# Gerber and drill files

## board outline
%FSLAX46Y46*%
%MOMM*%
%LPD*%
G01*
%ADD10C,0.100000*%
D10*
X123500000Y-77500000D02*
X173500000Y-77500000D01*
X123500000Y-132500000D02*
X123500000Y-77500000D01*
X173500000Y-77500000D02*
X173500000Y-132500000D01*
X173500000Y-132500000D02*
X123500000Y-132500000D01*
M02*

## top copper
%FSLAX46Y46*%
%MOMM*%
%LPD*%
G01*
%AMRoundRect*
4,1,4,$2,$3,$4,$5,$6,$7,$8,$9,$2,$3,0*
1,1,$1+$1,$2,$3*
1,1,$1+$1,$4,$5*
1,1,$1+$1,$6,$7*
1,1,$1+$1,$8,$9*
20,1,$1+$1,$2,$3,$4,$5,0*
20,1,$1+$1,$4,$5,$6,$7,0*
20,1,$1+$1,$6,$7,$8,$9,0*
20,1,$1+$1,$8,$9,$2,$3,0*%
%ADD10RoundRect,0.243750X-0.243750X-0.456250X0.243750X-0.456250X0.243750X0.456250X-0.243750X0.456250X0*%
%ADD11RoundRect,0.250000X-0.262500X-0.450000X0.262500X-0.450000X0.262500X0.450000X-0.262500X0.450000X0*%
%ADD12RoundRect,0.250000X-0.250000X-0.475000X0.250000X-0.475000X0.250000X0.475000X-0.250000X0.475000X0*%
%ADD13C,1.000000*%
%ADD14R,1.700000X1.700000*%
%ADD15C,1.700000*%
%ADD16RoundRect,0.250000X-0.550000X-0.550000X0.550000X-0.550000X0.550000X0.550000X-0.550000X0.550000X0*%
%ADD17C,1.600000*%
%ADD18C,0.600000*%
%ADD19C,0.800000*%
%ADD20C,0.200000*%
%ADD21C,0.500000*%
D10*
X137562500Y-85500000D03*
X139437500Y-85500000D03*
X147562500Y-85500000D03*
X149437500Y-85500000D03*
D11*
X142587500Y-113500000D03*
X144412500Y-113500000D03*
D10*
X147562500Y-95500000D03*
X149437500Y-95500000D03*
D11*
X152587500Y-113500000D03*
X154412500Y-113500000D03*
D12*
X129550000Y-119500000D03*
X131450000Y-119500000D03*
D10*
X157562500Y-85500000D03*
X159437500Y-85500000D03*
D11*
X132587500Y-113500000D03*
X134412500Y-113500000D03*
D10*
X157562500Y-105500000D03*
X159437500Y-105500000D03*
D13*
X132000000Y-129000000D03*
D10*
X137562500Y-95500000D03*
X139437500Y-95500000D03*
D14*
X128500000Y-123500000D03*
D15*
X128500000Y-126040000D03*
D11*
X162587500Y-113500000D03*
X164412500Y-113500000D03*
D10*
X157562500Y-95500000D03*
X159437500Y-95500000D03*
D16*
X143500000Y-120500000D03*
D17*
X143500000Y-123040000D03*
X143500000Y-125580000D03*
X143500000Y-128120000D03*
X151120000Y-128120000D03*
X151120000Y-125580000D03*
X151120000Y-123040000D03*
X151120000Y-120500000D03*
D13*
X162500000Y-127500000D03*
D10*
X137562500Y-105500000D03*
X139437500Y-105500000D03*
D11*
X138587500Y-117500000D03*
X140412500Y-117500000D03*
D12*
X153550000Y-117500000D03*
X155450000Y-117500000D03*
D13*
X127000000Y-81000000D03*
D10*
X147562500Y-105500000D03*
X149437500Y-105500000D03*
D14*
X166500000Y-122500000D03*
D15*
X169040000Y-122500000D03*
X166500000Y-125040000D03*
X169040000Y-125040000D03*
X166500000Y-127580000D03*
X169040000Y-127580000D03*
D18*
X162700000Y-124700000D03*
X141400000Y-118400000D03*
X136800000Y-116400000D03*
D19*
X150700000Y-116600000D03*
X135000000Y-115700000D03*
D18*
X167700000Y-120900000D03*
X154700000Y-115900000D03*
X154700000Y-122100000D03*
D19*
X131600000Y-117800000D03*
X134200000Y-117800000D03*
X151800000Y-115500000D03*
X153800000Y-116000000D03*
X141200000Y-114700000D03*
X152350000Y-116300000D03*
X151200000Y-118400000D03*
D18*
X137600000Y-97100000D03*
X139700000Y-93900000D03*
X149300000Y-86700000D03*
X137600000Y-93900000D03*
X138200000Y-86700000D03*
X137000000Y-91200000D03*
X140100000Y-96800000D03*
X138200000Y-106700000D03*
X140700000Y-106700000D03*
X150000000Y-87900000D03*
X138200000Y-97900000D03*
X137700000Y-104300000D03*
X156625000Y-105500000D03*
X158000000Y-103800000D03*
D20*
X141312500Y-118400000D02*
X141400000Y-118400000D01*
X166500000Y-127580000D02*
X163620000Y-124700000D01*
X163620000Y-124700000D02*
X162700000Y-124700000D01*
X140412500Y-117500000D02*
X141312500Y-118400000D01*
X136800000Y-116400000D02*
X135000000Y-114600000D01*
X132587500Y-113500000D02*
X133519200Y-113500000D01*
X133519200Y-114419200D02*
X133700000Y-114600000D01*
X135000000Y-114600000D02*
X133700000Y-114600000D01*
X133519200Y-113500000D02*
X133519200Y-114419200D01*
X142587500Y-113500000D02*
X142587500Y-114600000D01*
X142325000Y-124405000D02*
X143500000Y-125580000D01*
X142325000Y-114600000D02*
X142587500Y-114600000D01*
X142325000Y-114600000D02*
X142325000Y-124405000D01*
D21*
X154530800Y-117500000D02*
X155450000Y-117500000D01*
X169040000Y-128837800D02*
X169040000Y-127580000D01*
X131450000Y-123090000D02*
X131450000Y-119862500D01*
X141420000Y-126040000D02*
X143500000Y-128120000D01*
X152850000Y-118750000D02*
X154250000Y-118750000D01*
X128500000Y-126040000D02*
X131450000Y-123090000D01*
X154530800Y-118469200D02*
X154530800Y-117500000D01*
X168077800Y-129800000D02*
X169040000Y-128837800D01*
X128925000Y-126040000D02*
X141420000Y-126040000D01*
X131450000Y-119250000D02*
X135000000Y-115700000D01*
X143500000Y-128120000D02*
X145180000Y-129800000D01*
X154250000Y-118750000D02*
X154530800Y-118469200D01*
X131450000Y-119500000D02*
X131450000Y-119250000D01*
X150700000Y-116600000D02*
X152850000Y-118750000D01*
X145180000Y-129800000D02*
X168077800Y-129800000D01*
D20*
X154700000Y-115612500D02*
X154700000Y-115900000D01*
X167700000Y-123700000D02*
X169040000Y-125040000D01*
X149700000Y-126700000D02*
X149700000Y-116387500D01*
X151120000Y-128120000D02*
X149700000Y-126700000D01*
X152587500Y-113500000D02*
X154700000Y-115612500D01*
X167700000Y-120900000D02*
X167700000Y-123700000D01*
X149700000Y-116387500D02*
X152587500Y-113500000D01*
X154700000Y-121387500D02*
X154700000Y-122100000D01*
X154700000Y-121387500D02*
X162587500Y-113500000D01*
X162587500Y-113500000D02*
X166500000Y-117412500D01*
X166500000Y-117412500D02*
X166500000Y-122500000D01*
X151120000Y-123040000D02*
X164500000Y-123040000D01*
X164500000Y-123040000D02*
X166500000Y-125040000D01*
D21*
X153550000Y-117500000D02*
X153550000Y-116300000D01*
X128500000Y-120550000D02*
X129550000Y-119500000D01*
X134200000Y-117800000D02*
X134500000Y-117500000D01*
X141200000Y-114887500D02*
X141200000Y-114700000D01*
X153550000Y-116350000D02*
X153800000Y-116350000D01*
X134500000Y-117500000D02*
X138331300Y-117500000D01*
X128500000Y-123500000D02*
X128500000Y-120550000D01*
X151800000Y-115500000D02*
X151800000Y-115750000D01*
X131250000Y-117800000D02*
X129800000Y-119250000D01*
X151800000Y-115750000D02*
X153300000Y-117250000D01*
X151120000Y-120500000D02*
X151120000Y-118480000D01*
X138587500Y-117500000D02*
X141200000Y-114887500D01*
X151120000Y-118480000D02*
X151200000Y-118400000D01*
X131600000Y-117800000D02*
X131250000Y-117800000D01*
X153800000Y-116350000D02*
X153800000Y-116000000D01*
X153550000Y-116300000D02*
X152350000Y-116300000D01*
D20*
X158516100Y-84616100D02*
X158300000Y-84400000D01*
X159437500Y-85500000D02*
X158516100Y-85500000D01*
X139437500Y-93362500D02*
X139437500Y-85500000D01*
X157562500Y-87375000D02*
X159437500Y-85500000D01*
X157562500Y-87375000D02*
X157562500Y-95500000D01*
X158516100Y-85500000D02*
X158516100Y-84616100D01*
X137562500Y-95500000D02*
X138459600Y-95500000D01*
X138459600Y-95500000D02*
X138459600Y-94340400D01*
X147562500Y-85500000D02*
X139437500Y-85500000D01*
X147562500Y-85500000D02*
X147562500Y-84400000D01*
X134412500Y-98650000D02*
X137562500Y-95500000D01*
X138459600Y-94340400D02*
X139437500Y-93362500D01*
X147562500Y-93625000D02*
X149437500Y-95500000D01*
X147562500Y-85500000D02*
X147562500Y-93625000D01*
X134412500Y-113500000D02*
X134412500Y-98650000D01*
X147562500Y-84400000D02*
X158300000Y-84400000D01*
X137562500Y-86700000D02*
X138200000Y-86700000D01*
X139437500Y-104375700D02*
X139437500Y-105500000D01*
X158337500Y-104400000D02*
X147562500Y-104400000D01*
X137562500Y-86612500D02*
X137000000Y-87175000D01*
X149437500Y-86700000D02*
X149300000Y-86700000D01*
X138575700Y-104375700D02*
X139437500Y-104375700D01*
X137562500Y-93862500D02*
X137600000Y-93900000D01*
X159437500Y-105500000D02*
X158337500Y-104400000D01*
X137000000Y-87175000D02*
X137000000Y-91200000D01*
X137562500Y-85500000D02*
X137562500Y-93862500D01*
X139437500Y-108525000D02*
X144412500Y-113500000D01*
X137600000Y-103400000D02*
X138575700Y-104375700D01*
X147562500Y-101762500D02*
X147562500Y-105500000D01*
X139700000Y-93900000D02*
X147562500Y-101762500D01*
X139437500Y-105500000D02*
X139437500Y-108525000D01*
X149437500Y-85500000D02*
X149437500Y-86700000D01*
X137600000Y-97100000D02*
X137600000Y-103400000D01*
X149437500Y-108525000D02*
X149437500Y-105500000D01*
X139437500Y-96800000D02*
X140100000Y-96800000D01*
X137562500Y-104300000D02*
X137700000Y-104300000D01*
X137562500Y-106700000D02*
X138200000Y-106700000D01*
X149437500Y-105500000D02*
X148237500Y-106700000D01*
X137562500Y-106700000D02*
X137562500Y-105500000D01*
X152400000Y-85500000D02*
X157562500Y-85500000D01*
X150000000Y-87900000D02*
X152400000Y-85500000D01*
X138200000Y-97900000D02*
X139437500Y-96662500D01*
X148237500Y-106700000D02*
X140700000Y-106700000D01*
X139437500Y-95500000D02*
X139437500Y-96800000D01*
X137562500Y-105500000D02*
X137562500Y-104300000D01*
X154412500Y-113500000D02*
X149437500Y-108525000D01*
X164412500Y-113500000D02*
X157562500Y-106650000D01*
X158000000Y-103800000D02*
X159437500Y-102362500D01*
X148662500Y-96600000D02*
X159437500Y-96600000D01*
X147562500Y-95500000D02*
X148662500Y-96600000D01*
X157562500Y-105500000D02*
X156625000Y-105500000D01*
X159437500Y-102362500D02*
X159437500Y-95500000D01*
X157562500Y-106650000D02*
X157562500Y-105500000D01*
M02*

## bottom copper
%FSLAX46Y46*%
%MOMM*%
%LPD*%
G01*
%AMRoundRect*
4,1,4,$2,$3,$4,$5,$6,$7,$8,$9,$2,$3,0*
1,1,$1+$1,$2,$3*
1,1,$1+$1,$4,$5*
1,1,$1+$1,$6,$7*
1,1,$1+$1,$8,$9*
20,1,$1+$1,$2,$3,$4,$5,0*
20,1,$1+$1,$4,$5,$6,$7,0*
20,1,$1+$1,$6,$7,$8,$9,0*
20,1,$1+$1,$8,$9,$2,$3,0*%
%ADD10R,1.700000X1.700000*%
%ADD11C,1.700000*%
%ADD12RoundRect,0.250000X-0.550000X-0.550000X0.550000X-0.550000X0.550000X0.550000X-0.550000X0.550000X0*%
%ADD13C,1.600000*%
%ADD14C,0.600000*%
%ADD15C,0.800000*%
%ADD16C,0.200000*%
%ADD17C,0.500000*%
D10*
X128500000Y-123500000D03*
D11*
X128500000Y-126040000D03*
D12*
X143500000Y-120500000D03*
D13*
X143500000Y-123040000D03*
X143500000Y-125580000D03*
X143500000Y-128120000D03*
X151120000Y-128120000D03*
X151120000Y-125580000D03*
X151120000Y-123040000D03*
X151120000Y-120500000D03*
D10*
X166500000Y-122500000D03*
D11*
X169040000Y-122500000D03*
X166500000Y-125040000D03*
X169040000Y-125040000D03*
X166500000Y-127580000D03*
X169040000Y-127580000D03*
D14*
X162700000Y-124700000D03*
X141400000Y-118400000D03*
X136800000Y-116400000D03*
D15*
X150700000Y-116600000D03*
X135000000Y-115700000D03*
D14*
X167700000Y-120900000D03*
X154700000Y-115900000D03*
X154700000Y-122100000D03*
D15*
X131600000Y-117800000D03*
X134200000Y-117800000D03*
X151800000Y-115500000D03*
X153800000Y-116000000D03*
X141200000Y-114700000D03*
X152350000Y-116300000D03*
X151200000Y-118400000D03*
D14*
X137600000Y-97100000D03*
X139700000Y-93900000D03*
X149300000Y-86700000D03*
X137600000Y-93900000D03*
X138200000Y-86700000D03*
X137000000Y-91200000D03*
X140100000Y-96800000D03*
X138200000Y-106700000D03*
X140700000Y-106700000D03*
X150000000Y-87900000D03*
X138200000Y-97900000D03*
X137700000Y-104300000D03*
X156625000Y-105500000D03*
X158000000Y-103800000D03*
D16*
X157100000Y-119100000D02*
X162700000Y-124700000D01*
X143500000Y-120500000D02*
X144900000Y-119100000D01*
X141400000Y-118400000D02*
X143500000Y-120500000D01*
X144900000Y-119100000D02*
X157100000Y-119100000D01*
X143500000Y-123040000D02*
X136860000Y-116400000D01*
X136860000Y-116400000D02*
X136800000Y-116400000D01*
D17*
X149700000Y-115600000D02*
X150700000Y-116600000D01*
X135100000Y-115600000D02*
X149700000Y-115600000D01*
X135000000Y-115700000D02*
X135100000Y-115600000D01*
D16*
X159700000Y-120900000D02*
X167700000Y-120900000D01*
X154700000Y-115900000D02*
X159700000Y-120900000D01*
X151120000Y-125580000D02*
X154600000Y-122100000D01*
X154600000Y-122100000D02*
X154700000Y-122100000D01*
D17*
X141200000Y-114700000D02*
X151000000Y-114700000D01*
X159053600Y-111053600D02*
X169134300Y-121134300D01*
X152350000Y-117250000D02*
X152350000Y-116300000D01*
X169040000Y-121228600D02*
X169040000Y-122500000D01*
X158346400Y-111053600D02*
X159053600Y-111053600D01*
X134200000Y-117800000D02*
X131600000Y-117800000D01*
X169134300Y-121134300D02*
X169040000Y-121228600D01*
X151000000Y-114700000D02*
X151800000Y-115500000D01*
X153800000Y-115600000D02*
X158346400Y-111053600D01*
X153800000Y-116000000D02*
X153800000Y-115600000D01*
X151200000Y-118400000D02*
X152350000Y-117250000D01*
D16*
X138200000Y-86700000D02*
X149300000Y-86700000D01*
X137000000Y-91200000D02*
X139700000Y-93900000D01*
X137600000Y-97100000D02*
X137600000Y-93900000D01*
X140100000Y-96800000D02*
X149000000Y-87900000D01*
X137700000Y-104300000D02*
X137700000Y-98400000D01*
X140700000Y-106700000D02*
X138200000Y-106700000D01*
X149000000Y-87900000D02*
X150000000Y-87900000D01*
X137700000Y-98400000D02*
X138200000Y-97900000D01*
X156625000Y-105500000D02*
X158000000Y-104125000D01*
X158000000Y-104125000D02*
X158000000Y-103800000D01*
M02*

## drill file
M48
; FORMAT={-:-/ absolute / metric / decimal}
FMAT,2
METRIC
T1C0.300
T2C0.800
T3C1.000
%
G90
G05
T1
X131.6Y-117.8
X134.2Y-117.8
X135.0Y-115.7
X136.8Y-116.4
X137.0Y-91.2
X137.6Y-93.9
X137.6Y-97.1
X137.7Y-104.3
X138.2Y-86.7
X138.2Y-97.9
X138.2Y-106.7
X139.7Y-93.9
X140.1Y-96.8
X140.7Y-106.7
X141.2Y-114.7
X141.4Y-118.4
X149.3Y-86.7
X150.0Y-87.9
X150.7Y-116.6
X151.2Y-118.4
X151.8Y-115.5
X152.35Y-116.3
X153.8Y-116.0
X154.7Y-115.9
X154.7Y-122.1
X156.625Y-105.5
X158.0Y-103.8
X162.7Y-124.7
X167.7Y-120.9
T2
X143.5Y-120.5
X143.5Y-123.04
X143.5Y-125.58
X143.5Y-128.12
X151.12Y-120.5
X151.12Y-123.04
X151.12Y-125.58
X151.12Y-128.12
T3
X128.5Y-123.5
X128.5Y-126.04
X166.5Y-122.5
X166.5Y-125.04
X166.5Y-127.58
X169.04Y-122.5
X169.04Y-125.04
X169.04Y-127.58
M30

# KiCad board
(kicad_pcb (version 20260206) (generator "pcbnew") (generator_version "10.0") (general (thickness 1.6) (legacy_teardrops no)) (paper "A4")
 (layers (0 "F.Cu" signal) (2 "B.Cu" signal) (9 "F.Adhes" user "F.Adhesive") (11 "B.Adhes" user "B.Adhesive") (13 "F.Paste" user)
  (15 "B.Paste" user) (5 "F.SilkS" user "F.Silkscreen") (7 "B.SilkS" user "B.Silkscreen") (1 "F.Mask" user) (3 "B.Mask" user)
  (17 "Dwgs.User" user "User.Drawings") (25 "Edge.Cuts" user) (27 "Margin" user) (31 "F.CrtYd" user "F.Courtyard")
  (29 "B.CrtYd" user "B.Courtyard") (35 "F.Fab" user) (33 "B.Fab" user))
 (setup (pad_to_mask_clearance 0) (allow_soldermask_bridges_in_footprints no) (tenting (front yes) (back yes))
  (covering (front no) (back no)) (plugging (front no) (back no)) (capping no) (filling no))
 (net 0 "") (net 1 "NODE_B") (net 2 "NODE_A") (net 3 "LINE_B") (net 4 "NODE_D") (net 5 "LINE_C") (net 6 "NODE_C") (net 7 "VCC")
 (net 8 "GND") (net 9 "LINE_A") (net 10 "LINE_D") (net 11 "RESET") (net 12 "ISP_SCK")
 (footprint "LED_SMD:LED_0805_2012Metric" (layer "F.Cu") (at 138.5 85.5)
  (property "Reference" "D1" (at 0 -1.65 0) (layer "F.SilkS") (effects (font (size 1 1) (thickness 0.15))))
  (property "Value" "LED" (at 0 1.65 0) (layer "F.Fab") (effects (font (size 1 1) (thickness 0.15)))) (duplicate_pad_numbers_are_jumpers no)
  (pad "1" smd roundrect (at -0.9375 0) (size 0.975 1.4) (layers "F.Cu" "F.Mask" "F.Paste") (roundrect_rratio 0.25) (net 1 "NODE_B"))
  (pad "2" smd roundrect (at 0.9375 0) (size 0.975 1.4) (layers "F.Cu" "F.Mask" "F.Paste") (roundrect_rratio 0.25) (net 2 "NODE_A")))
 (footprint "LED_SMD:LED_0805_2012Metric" (layer "F.Cu") (at 148.5 85.5)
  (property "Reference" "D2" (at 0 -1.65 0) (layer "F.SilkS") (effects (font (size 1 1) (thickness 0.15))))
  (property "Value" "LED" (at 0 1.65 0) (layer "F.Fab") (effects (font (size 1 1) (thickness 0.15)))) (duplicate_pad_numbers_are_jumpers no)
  (pad "1" smd roundrect (at -0.9375 0) (size 0.975 1.4) (layers "F.Cu" "F.Mask" "F.Paste") (roundrect_rratio 0.25) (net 2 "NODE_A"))
  (pad "2" smd roundrect (at 0.9375 0) (size 0.975 1.4) (layers "F.Cu" "F.Mask" "F.Paste") (roundrect_rratio 0.25) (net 1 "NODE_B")))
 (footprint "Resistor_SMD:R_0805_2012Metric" (layer "F.Cu") (at 143.5 113.5)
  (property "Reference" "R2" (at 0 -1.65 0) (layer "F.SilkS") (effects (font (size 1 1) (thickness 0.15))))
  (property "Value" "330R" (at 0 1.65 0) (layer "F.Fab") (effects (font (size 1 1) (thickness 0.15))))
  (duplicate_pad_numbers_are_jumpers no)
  (pad "1" smd roundrect (at -0.9125 0) (size 1.025 1.4) (layers "F.Cu" "F.Mask" "F.Paste") (roundrect_rratio 0.243902) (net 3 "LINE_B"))
  (pad "2" smd roundrect (at 0.9125 0) (size 1.025 1.4) (layers "F.Cu" "F.Mask" "F.Paste") (roundrect_rratio 0.243902) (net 1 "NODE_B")))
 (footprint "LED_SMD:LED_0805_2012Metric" (layer "F.Cu") (at 148.5 95.5)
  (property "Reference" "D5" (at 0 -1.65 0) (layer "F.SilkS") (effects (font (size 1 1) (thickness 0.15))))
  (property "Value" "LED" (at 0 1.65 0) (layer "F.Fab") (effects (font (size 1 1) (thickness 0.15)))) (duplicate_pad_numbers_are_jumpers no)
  (pad "1" smd roundrect (at -0.9375 0) (size 0.975 1.4) (layers "F.Cu" "F.Mask" "F.Paste") (roundrect_rratio 0.25) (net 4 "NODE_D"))
  (pad "2" smd roundrect (at 0.9375 0) (size 0.975 1.4) (layers "F.Cu" "F.Mask" "F.Paste") (roundrect_rratio 0.25) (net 2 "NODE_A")))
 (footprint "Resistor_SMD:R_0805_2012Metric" (layer "F.Cu") (at 153.5 113.5)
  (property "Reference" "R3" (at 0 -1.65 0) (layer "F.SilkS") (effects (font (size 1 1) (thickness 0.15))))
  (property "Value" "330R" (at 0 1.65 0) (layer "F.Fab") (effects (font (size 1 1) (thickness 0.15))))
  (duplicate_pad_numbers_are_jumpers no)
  (pad "1" smd roundrect (at -0.9125 0) (size 1.025 1.4) (layers "F.Cu" "F.Mask" "F.Paste") (roundrect_rratio 0.243902) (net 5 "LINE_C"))
  (pad "2" smd roundrect (at 0.9125 0) (size 1.025 1.4) (layers "F.Cu" "F.Mask" "F.Paste") (roundrect_rratio 0.243902) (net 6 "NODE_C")))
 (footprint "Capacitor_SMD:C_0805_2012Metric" (layer "F.Cu") (at 130.5 119.5)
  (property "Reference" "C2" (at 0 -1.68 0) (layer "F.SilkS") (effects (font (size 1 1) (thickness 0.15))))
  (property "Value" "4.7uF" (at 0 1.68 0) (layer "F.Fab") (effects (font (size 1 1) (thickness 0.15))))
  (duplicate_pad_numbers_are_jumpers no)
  (pad "1" smd roundrect (at -0.95 0) (size 1 1.45) (layers "F.Cu" "F.Mask" "F.Paste") (roundrect_rratio 0.25) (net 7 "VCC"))
  (pad "2" smd roundrect (at 0.95 0) (size 1 1.45) (layers "F.Cu" "F.Mask" "F.Paste") (roundrect_rratio 0.25) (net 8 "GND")))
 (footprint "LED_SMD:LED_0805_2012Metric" (layer "F.Cu") (at 158.5 85.5)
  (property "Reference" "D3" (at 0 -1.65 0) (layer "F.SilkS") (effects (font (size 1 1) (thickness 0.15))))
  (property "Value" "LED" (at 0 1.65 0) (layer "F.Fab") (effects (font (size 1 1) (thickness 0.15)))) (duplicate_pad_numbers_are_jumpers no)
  (pad "1" smd roundrect (at -0.9375 0) (size 0.975 1.4) (layers "F.Cu" "F.Mask" "F.Paste") (roundrect_rratio 0.25) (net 6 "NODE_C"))
  (pad "2" smd roundrect (at 0.9375 0) (size 0.975 1.4) (layers "F.Cu" "F.Mask" "F.Paste") (roundrect_rratio 0.25) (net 2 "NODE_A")))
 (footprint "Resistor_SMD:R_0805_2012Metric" (layer "F.Cu") (at 133.5 113.5)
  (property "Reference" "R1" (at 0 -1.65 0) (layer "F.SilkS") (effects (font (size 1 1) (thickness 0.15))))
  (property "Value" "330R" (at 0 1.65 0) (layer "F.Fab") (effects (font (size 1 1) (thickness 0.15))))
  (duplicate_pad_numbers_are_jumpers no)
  (pad "1" smd roundrect (at -0.9125 0) (size 1.025 1.4) (layers "F.Cu" "F.Mask" "F.Paste") (roundrect_rratio 0.243902) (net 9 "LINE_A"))
  (pad "2" smd roundrect (at 0.9125 0) (size 1.025 1.4) (layers "F.Cu" "F.Mask" "F.Paste") (roundrect_rratio 0.243902) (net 2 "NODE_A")))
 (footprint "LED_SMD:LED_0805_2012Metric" (layer "F.Cu") (at 158.5 105.5)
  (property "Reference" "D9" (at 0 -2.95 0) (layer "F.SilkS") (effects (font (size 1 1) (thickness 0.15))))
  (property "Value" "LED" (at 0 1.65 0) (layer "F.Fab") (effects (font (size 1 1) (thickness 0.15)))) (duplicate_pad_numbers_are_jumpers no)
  (pad "1" smd roundrect (at -0.9375 0) (size 0.975 1.4) (layers "F.Cu" "F.Mask" "F.Paste") (roundrect_rratio 0.25) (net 4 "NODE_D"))
  (pad "2" smd roundrect (at 0.9375 0) (size 0.975 1.4) (layers "F.Cu" "F.Mask" "F.Paste") (roundrect_rratio 0.25) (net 1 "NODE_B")))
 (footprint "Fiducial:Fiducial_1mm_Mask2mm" (layer "F.Cu") (at 132 129)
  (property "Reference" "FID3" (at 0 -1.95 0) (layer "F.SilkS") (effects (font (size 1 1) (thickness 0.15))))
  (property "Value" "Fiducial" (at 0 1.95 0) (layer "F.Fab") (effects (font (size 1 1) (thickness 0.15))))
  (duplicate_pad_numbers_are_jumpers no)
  (pad "" smd circle (at 0 0) (size 1 1) (layers "F.Cu" "F.Mask") (solder_mask_margin 0.5) (clearance 0.6)))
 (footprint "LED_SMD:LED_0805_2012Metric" (layer "F.Cu") (at 138.5 95.5)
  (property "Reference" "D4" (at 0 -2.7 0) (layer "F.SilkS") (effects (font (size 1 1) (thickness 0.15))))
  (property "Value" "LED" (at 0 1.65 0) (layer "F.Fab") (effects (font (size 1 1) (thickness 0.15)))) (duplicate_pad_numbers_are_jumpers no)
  (pad "1" smd roundrect (at -0.9375 0) (size 0.975 1.4) (layers "F.Cu" "F.Mask" "F.Paste") (roundrect_rratio 0.25) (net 2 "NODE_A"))
  (pad "2" smd roundrect (at 0.9375 0) (size 0.975 1.4) (layers "F.Cu" "F.Mask" "F.Paste") (roundrect_rratio 0.25) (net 6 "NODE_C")))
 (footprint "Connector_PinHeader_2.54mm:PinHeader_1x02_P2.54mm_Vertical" (layer "F.Cu") (at 128.5 123.5)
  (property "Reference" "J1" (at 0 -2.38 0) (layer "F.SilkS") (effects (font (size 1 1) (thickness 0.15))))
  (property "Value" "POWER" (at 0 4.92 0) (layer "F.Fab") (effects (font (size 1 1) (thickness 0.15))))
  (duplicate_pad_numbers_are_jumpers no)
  (pad "1" thru_hole rect (at 0 0) (size 1.7 1.7) (drill 1) (layers "*.Cu" "*.Mask") (remove_unused_layers no) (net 7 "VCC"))
  (pad "2" thru_hole circle (at 0 2.54) (size 1.7 1.7) (drill 1) (layers "*.Cu" "*.Mask") (remove_unused_layers no) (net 8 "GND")))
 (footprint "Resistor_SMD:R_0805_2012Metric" (layer "F.Cu") (at 163.5 113.5)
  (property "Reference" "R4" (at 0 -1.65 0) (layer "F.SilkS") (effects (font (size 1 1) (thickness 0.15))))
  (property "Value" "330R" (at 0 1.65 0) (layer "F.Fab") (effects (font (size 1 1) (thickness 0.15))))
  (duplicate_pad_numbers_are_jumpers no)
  (pad "1" smd roundrect (at -0.9125 0) (size 1.025 1.4) (layers "F.Cu" "F.Mask" "F.Paste") (roundrect_rratio 0.243902) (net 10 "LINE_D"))
  (pad "2" smd roundrect (at 0.9125 0) (size 1.025 1.4) (layers "F.Cu" "F.Mask" "F.Paste") (roundrect_rratio 0.243902) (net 4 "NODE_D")))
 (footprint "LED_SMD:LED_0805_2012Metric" (layer "F.Cu") (at 158.5 95.5)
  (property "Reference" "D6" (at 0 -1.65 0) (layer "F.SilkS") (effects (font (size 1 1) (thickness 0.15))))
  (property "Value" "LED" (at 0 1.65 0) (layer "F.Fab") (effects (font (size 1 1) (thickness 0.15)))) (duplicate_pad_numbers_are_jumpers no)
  (pad "1" smd roundrect (at -0.9375 0) (size 0.975 1.4) (layers "F.Cu" "F.Mask" "F.Paste") (roundrect_rratio 0.25) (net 2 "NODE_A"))
  (pad "2" smd roundrect (at 0.9375 0) (size 0.975 1.4) (layers "F.Cu" "F.Mask" "F.Paste") (roundrect_rratio 0.25) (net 4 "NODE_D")))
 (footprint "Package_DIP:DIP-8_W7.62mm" (layer "F.Cu") (at 143.5 120.5)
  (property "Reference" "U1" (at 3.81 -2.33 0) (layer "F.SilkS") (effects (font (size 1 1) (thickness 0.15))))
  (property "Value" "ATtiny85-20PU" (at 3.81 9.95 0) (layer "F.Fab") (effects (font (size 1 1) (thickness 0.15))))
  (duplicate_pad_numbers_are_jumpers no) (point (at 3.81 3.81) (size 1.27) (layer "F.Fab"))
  (pad "1" thru_hole roundrect (at 0 0) (size 1.6 1.6) (drill 0.8) (layers "*.Cu" "*.Mask") (remove_unused_layers no)
   (roundrect_rratio 0.15625) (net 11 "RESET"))
  (pad "2" thru_hole circle (at 0 2.54) (size 1.6 1.6) (drill 0.8) (layers "*.Cu" "*.Mask") (remove_unused_layers no) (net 9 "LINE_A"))
  (pad "3" thru_hole circle (at 0 5.08) (size 1.6 1.6) (drill 0.8) (layers "*.Cu" "*.Mask") (remove_unused_layers no) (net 3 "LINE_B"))
  (pad "4" thru_hole circle (at 0 7.62) (size 1.6 1.6) (drill 0.8) (layers "*.Cu" "*.Mask") (remove_unused_layers no) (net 8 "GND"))
  (pad "5" thru_hole circle (at 7.62 7.62) (size 1.6 1.6) (drill 0.8) (layers "*.Cu" "*.Mask") (remove_unused_layers no) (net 5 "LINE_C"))
  (pad "6" thru_hole circle (at 7.62 5.08) (size 1.6 1.6) (drill 0.8) (layers "*.Cu" "*.Mask") (remove_unused_layers no) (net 10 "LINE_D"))
  (pad "7" thru_hole circle (at 7.62 2.54) (size 1.6 1.6) (drill 0.8) (layers "*.Cu" "*.Mask") (remove_unused_layers no) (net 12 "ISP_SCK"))
  (pad "8" thru_hole circle (at 7.62 0) (size 1.6 1.6) (drill 0.8) (layers "*.Cu" "*.Mask") (remove_unused_layers no) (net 7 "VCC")))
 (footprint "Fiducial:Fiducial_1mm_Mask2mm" (layer "F.Cu") (at 162.5 127.5)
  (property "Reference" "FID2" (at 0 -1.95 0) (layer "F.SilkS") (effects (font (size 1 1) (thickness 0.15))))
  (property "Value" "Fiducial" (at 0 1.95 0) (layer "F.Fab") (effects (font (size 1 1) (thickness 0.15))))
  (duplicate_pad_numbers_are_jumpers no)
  (pad "" smd circle (at 0 0) (size 1 1) (layers "F.Cu" "F.Mask") (solder_mask_margin 0.5) (clearance 0.6)))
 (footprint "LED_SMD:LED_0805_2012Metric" (layer "F.Cu") (at 138.5 105.5)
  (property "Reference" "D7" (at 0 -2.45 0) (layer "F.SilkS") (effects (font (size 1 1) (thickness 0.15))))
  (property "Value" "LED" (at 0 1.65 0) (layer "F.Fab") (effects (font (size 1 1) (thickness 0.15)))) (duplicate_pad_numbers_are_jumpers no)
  (pad "1" smd roundrect (at -0.9375 0) (size 0.975 1.4) (layers "F.Cu" "F.Mask" "F.Paste") (roundrect_rratio 0.25) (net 6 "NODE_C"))
  (pad "2" smd roundrect (at 0.9375 0) (size 0.975 1.4) (layers "F.Cu" "F.Mask" "F.Paste") (roundrect_rratio 0.25) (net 1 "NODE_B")))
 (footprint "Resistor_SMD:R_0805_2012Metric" (layer "F.Cu") (at 139.5 117.5)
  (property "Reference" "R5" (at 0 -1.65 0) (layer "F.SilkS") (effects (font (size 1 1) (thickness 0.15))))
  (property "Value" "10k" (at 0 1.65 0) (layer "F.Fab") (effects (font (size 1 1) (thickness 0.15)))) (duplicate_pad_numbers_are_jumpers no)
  (pad "1" smd roundrect (at -0.9125 0) (size 1.025 1.4) (layers "F.Cu" "F.Mask" "F.Paste") (roundrect_rratio 0.243902) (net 7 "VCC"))
  (pad "2" smd roundrect (at 0.9125 0) (size 1.025 1.4) (layers "F.Cu" "F.Mask" "F.Paste") (roundrect_rratio 0.243902) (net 11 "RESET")))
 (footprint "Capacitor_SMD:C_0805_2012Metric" (layer "F.Cu") (at 154.5 117.5)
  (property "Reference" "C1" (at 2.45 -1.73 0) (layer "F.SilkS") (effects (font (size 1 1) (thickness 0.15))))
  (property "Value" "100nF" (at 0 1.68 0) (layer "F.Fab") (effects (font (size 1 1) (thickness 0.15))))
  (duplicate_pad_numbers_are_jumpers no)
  (pad "1" smd roundrect (at -0.95 0) (size 1 1.45) (layers "F.Cu" "F.Mask" "F.Paste") (roundrect_rratio 0.25) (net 7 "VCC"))
  (pad "2" smd roundrect (at 0.95 0) (size 1 1.45) (layers "F.Cu" "F.Mask" "F.Paste") (roundrect_rratio 0.25) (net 8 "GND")))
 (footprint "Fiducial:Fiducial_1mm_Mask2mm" (layer "F.Cu") (at 127 81)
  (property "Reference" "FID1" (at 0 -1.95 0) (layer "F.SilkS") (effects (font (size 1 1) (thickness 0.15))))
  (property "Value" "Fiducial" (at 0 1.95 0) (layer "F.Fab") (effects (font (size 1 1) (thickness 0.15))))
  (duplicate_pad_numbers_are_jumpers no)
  (pad "" smd circle (at 0 0) (size 1 1) (layers "F.Cu" "F.Mask") (solder_mask_margin 0.5) (clearance 0.6)))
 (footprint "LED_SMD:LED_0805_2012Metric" (layer "F.Cu") (at 148.5 105.5)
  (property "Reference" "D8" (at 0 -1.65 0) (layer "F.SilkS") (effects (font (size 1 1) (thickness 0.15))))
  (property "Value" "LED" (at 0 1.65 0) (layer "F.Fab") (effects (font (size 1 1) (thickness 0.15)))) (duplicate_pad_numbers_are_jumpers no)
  (pad "1" smd roundrect (at -0.9375 0) (size 0.975 1.4) (layers "F.Cu" "F.Mask" "F.Paste") (roundrect_rratio 0.25) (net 1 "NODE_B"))
  (pad "2" smd roundrect (at 0.9375 0) (size 0.975 1.4) (layers "F.Cu" "F.Mask" "F.Paste") (roundrect_rratio 0.25) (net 6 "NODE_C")))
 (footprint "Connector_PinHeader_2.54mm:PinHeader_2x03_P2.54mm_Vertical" (layer "F.Cu") (at 166.5 122.5)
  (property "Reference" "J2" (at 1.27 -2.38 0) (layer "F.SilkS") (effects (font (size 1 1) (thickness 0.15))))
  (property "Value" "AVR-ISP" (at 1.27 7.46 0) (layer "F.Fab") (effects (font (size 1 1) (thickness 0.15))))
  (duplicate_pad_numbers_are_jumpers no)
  (pad "1" thru_hole rect (at 0 0) (size 1.7 1.7) (drill 1) (layers "*.Cu" "*.Mask") (remove_unused_layers no) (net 10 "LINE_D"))
  (pad "2" thru_hole circle (at 2.54 0) (size 1.7 1.7) (drill 1) (layers "*.Cu" "*.Mask") (remove_unused_layers no) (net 7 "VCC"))
  (pad "3" thru_hole circle (at 0 2.54) (size 1.7 1.7) (drill 1) (layers "*.Cu" "*.Mask") (remove_unused_layers no) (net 12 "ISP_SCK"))
  (pad "4" thru_hole circle (at 2.54 2.54) (size 1.7 1.7) (drill 1) (layers "*.Cu" "*.Mask") (remove_unused_layers no) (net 5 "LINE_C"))
  (pad "5" thru_hole circle (at 0 5.08) (size 1.7 1.7) (drill 1) (layers "*.Cu" "*.Mask") (remove_unused_layers no) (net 11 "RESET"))
  (pad "6" thru_hole circle (at 2.54 5.08) (size 1.7 1.7) (drill 1) (layers "*.Cu" "*.Mask") (remove_unused_layers no) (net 8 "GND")))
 (gr_line (start 123.5 77.5) (end 173.5 77.5) (stroke (width 0.1) (type default)) (layer "Edge.Cuts"))
 (gr_line (start 123.5 132.5) (end 123.5 77.5) (stroke (width 0.1) (type default)) (layer "Edge.Cuts"))
 (gr_line (start 173.5 77.5) (end 173.5 132.5) (stroke (width 0.1) (type default)) (layer "Edge.Cuts"))
 (gr_line (start 173.5 132.5) (end 123.5 132.5) (stroke (width 0.1) (type default)) (layer "Edge.Cuts"))
 (segment (start 141.3125 118.4) (end 141.4 118.4) (width 0.2) (layer "F.Cu") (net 11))
 (segment (start 166.5 127.58) (end 163.62 124.7) (width 0.2) (layer "F.Cu") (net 11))
 (segment (start 163.62 124.7) (end 162.7 124.7) (width 0.2) (layer "F.Cu") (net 11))
 (segment (start 140.4125 117.5) (end 141.3125 118.4) (width 0.2) (layer "F.Cu") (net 11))
 (via (at 162.7 124.7) (size 0.6) (drill 0.3) (layers "F.Cu" "B.Cu") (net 11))
 (via (at 141.4 118.4) (size 0.6) (drill 0.3) (layers "F.Cu" "B.Cu") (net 11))
 (segment (start 157.1 119.1) (end 162.7 124.7) (width 0.2) (layer "B.Cu") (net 11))
 (segment (start 143.5 120.5) (end 144.9 119.1) (width 0.2) (layer "B.Cu") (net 11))
 (segment (start 141.4 118.4) (end 143.5 120.5) (width 0.2) (layer "B.Cu") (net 11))
 (segment (start 144.9 119.1) (end 157.1 119.1) (width 0.2) (layer "B.Cu") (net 11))
 (segment (start 136.8 116.4) (end 135 114.6) (width 0.2) (layer "F.Cu") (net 9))
 (segment (start 132.5875 113.5) (end 133.5192 113.5) (width 0.2) (layer "F.Cu") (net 9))
 (segment (start 133.5192 114.4192) (end 133.7 114.6) (width 0.2) (layer "F.Cu") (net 9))
 (segment (start 135 114.6) (end 133.7 114.6) (width 0.2) (layer "F.Cu") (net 9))
 (segment (start 133.5192 113.5) (end 133.5192 114.4192) (width 0.2) (layer "F.Cu") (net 9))
 (via (at 136.8 116.4) (size 0.6) (drill 0.3) (layers "F.Cu" "B.Cu") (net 9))
 (segment (start 143.5 123.04) (end 136.86 116.4) (width 0.2) (layer "B.Cu") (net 9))
 (segment (start 136.86 116.4) (end 136.8 116.4) (width 0.2) (layer "B.Cu") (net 9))
 (segment (start 142.5875 113.5) (end 142.5875 114.6) (width 0.2) (layer "F.Cu") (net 3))
 (segment (start 142.325 124.405) (end 143.5 125.58) (width 0.2) (layer "F.Cu") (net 3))
 (segment (start 142.325 114.6) (end 142.5875 114.6) (width 0.2) (layer "F.Cu") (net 3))
 (segment (start 142.325 114.6) (end 142.325 124.405) (width 0.2) (layer "F.Cu") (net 3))
 (segment (start 154.5308 117.5) (end 155.45 117.5) (width 0.5) (layer "F.Cu") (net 8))
 (segment (start 169.04 128.8378) (end 169.04 127.58) (width 0.5) (layer "F.Cu") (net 8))
 (segment (start 131.45 123.09) (end 131.45 119.8625) (width 0.5) (layer "F.Cu") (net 8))
 (segment (start 141.42 126.04) (end 143.5 128.12) (width 0.5) (layer "F.Cu") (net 8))
 (segment (start 152.85 118.75) (end 154.25 118.75) (width 0.5) (layer "F.Cu") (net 8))
 (segment (start 128.5 126.04) (end 131.45 123.09) (width 0.5) (layer "F.Cu") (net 8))
 (segment (start 154.5308 118.4692) (end 154.5308 117.5) (width 0.5) (layer "F.Cu") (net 8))
 (segment (start 168.0778 129.8) (end 169.04 128.8378) (width 0.5) (layer "F.Cu") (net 8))
 (segment (start 128.925 126.04) (end 141.42 126.04) (width 0.5) (layer "F.Cu") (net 8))
 (segment (start 131.45 119.25) (end 135 115.7) (width 0.5) (layer "F.Cu") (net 8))
 (segment (start 143.5 128.12) (end 145.18 129.8) (width 0.5) (layer "F.Cu") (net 8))
 (segment (start 154.25 118.75) (end 154.5308 118.4692) (width 0.5) (layer "F.Cu") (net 8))
 (segment (start 131.45 119.5) (end 131.45 119.25) (width 0.5) (layer "F.Cu") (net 8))
 (segment (start 150.7 116.6) (end 152.85 118.75) (width 0.5) (layer "F.Cu") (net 8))
 (segment (start 145.18 129.8) (end 168.0778 129.8) (width 0.5) (layer "F.Cu") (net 8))
 (via (at 150.7 116.6) (size 0.8) (drill 0.3) (layers "F.Cu" "B.Cu") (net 8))
 (via (at 135 115.7) (size 0.8) (drill 0.3) (layers "F.Cu" "B.Cu") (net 8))
 (segment (start 149.7 115.6) (end 150.7 116.6) (width 0.5) (layer "B.Cu") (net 8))
 (segment (start 135.1 115.6) (end 149.7 115.6) (width 0.5) (layer "B.Cu") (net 8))
 (segment (start 135 115.7) (end 135.1 115.6) (width 0.5) (layer "B.Cu") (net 8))
 (segment (start 154.7 115.6125) (end 154.7 115.9) (width 0.2) (layer "F.Cu") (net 5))
 (segment (start 167.7 123.7) (end 169.04 125.04) (width 0.2) (layer "F.Cu") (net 5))
 (segment (start 149.7 126.7) (end 149.7 116.3875) (width 0.2) (layer "F.Cu") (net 5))
 (segment (start 151.12 128.12) (end 149.7 126.7) (width 0.2) (layer "F.Cu") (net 5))
 (segment (start 152.5875 113.5) (end 154.7 115.6125) (width 0.2) (layer "F.Cu") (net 5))
 (segment (start 167.7 120.9) (end 167.7 123.7) (width 0.2) (layer "F.Cu") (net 5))
 (segment (start 149.7 116.3875) (end 152.5875 113.5) (width 0.2) (layer "F.Cu") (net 5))
 (via (at 167.7 120.9) (size 0.6) (drill 0.3) (layers "F.Cu" "B.Cu") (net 5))
 (via (at 154.7 115.9) (size 0.6) (drill 0.3) (layers "F.Cu" "B.Cu") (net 5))
 (segment (start 159.7 120.9) (end 167.7 120.9) (width 0.2) (layer "B.Cu") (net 5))
 (segment (start 154.7 115.9) (end 159.7 120.9) (width 0.2) (layer "B.Cu") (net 5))
 (segment (start 154.7 121.3875) (end 154.7 122.1) (width 0.2) (layer "F.Cu") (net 10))
 (segment (start 154.7 121.3875) (end 162.5875 113.5) (width 0.2) (layer "F.Cu") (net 10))
 (segment (start 162.5875 113.5) (end 166.5 117.4125) (width 0.2) (layer "F.Cu") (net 10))
 (segment (start 166.5 117.4125) (end 166.5 122.5) (width 0.2) (layer "F.Cu") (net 10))
 (via (at 154.7 122.1) (size 0.6) (drill 0.3) (layers "F.Cu" "B.Cu") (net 10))
 (segment (start 151.12 125.58) (end 154.6 122.1) (width 0.2) (layer "B.Cu") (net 10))
 (segment (start 154.6 122.1) (end 154.7 122.1) (width 0.2) (layer "B.Cu") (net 10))
 (segment (start 151.12 123.04) (end 164.5 123.04) (width 0.2) (layer "F.Cu") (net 12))
 (segment (start 164.5 123.04) (end 166.5 125.04) (width 0.2) (layer "F.Cu") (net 12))
 (segment (start 153.55 117.5) (end 153.55 116.3) (width 0.5) (layer "F.Cu") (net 7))
 (segment (start 128.5 120.55) (end 129.55 119.5) (width 0.5) (layer "F.Cu") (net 7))
 (segment (start 134.2 117.8) (end 134.5 117.5) (width 0.5) (layer "F.Cu") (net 7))
 (segment (start 141.2 114.8875) (end 141.2 114.7) (width 0.5) (layer "F.Cu") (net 7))
 (segment (start 153.55 116.35) (end 153.8 116.35) (width 0.5) (layer "F.Cu") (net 7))
 (segment (start 134.5 117.5) (end 138.3313 117.5) (width 0.5) (layer "F.Cu") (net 7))
 (segment (start 128.5 123.5) (end 128.5 120.55) (width 0.5) (layer "F.Cu") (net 7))
 (segment (start 151.8 115.5) (end 151.8 115.75) (width 0.5) (layer "F.Cu") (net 7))
 (segment (start 131.25 117.8) (end 129.8 119.25) (width 0.5) (layer "F.Cu") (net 7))
 (segment (start 151.8 115.75) (end 153.3 117.25) (width 0.5) (layer "F.Cu") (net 7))
 (segment (start 151.12 120.5) (end 151.12 118.48) (width 0.5) (layer "F.Cu") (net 7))
 (segment (start 138.5875 117.5) (end 141.2 114.8875) (width 0.5) (layer "F.Cu") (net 7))
 (segment (start 151.12 118.48) (end 151.2 118.4) (width 0.5) (layer "F.Cu") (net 7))
 (segment (start 131.6 117.8) (end 131.25 117.8) (width 0.5) (layer "F.Cu") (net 7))
 (segment (start 153.8 116.35) (end 153.8 116) (width 0.5) (layer "F.Cu") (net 7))
 (segment (start 153.55 116.3) (end 152.35 116.3) (width 0.5) (layer "F.Cu") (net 7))
 (via (at 131.6 117.8) (size 0.8) (drill 0.3) (layers "F.Cu" "B.Cu") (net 7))
 (via (at 134.2 117.8) (size 0.8) (drill 0.3) (layers "F.Cu" "B.Cu") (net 7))
 (via (at 151.8 115.5) (size 0.8) (drill 0.3) (layers "F.Cu" "B.Cu") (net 7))
 (via (at 153.8 116) (size 0.8) (drill 0.3) (layers "F.Cu" "B.Cu") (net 7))
 (via (at 141.2 114.7) (size 0.8) (drill 0.3) (layers "F.Cu" "B.Cu") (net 7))
 (via (at 152.35 116.3) (size 0.8) (drill 0.3) (layers "F.Cu" "B.Cu") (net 7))
 (via (at 151.2 118.4) (size 0.8) (drill 0.3) (layers "F.Cu" "B.Cu") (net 7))
 (segment (start 141.2 114.7) (end 151 114.7) (width 0.5) (layer "B.Cu") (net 7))
 (segment (start 159.0536 111.0536) (end 169.1343 121.1343) (width 0.5) (layer "B.Cu") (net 7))
 (segment (start 152.35 117.25) (end 152.35 116.3) (width 0.5) (layer "B.Cu") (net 7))
 (segment (start 169.04 121.2286) (end 169.04 122.5) (width 0.5) (layer "B.Cu") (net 7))
 (segment (start 158.3464 111.0536) (end 159.0536 111.0536) (width 0.5) (layer "B.Cu") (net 7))
 (segment (start 134.2 117.8) (end 131.6 117.8) (width 0.5) (layer "B.Cu") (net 7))
 (segment (start 169.1343 121.1343) (end 169.04 121.2286) (width 0.5) (layer "B.Cu") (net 7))
 (segment (start 151 114.7) (end 151.8 115.5) (width 0.5) (layer "B.Cu") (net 7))
 (segment (start 153.8 115.6) (end 158.3464 111.0536) (width 0.5) (layer "B.Cu") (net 7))
 (segment (start 153.8 116) (end 153.8 115.6) (width 0.5) (layer "B.Cu") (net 7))
 (segment (start 151.2 118.4) (end 152.35 117.25) (width 0.5) (layer "B.Cu") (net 7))
 (segment (start 158.5161 84.6161) (end 158.3 84.4) (width 0.2) (layer "F.Cu") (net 2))
 (segment (start 159.4375 85.5) (end 158.5161 85.5) (width 0.2) (layer "F.Cu") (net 2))
 (segment (start 139.4375 93.3625) (end 139.4375 85.5) (width 0.2) (layer "F.Cu") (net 2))
 (segment (start 157.5625 87.375) (end 159.4375 85.5) (width 0.2) (layer "F.Cu") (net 2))
 (segment (start 157.5625 87.375) (end 157.5625 95.5) (width 0.2) (layer "F.Cu") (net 2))
 (segment (start 158.5161 85.5) (end 158.5161 84.6161) (width 0.2) (layer "F.Cu") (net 2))
 (segment (start 137.5625 95.5) (end 138.4596 95.5) (width 0.2) (layer "F.Cu") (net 2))
 (segment (start 138.4596 95.5) (end 138.4596 94.3404) (width 0.2) (layer "F.Cu") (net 2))
 (segment (start 147.5625 85.5) (end 139.4375 85.5) (width 0.2) (layer "F.Cu") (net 2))
 (segment (start 147.5625 85.5) (end 147.5625 84.4) (width 0.2) (layer "F.Cu") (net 2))
 (segment (start 134.4125 98.65) (end 137.5625 95.5) (width 0.2) (layer "F.Cu") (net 2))
 (segment (start 138.4596 94.3404) (end 139.4375 93.3625) (width 0.2) (layer "F.Cu") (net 2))
 (segment (start 147.5625 93.625) (end 149.4375 95.5) (width 0.2) (layer "F.Cu") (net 2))
 (segment (start 147.5625 85.5) (end 147.5625 93.625) (width 0.2) (layer "F.Cu") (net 2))
 (segment (start 134.4125 113.5) (end 134.4125 98.65) (width 0.2) (layer "F.Cu") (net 2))
 (segment (start 147.5625 84.4) (end 158.3 84.4) (width 0.2) (layer "F.Cu") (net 2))
 (segment (start 137.5625 86.7) (end 138.2 86.7) (width 0.2) (layer "F.Cu") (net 1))
 (segment (start 139.4375 104.3757) (end 139.4375 105.5) (width 0.2) (layer "F.Cu") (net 1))
 (segment (start 158.3375 104.4) (end 147.5625 104.4) (width 0.2) (layer "F.Cu") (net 1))
 (segment (start 137.5625 86.6125) (end 137 87.175) (width 0.2) (layer "F.Cu") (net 1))
 (segment (start 149.4375 86.7) (end 149.3 86.7) (width 0.2) (layer "F.Cu") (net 1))
 (segment (start 138.5757 104.3757) (end 139.4375 104.3757) (width 0.2) (layer "F.Cu") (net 1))
 (segment (start 137.5625 93.8625) (end 137.6 93.9) (width 0.2) (layer "F.Cu") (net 1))
 (segment (start 159.4375 105.5) (end 158.3375 104.4) (width 0.2) (layer "F.Cu") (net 1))
 (segment (start 137 87.175) (end 137 91.2) (width 0.2) (layer "F.Cu") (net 1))
 (segment (start 137.5625 85.5) (end 137.5625 93.8625) (width 0.2) (layer "F.Cu") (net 1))
 (segment (start 139.4375 108.525) (end 144.4125 113.5) (width 0.2) (layer "F.Cu") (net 1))
 (segment (start 137.6 103.4) (end 138.5757 104.3757) (width 0.2) (layer "F.Cu") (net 1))
 (segment (start 147.5625 101.7625) (end 147.5625 105.5) (width 0.2) (layer "F.Cu") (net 1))
 (segment (start 139.7 93.9) (end 147.5625 101.7625) (width 0.2) (layer "F.Cu") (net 1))
 (segment (start 139.4375 105.5) (end 139.4375 108.525) (width 0.2) (layer "F.Cu") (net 1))
 (segment (start 149.4375 85.5) (end 149.4375 86.7) (width 0.2) (layer "F.Cu") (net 1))
 (segment (start 137.6 97.1) (end 137.6 103.4) (width 0.2) (layer "F.Cu") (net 1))
 (via (at 137.6 97.1) (size 0.6) (drill 0.3) (layers "F.Cu" "B.Cu") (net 1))
 (via (at 139.7 93.9) (size 0.6) (drill 0.3) (layers "F.Cu" "B.Cu") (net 1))
 (via (at 149.3 86.7) (size 0.6) (drill 0.3) (layers "F.Cu" "B.Cu") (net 1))
 (via (at 137.6 93.9) (size 0.6) (drill 0.3) (layers "F.Cu" "B.Cu") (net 1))
 (via (at 138.2 86.7) (size 0.6) (drill 0.3) (layers "F.Cu" "B.Cu") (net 1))
 (via (at 137 91.2) (size 0.6) (drill 0.3) (layers "F.Cu" "B.Cu") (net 1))
 (segment (start 138.2 86.7) (end 149.3 86.7) (width 0.2) (layer "B.Cu") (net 1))
 (segment (start 137 91.2) (end 139.7 93.9) (width 0.2) (layer "B.Cu") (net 1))
 (segment (start 137.6 97.1) (end 137.6 93.9) (width 0.2) (layer "B.Cu") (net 1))
 (segment (start 149.4375 108.525) (end 149.4375 105.5) (width 0.2) (layer "F.Cu") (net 6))
 (segment (start 139.4375 96.8) (end 140.1 96.8) (width 0.2) (layer "F.Cu") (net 6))
 (segment (start 137.5625 104.3) (end 137.7 104.3) (width 0.2) (layer "F.Cu") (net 6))
 (segment (start 137.5625 106.7) (end 138.2 106.7) (width 0.2) (layer "F.Cu") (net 6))
 (segment (start 149.4375 105.5) (end 148.2375 106.7) (width 0.2) (layer "F.Cu") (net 6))
 (segment (start 137.5625 106.7) (end 137.5625 105.5) (width 0.2) (layer "F.Cu") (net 6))
 (segment (start 152.4 85.5) (end 157.5625 85.5) (width 0.2) (layer "F.Cu") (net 6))
 (segment (start 150 87.9) (end 152.4 85.5) (width 0.2) (layer "F.Cu") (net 6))
 (segment (start 138.2 97.9) (end 139.4375 96.6625) (width 0.2) (layer "F.Cu") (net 6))
 (segment (start 148.2375 106.7) (end 140.7 106.7) (width 0.2) (layer "F.Cu") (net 6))
 (segment (start 139.4375 95.5) (end 139.4375 96.8) (width 0.2) (layer "F.Cu") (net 6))
 (segment (start 137.5625 105.5) (end 137.5625 104.3) (width 0.2) (layer "F.Cu") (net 6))
 (segment (start 154.4125 113.5) (end 149.4375 108.525) (width 0.2) (layer "F.Cu") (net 6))
 (via (at 140.1 96.8) (size 0.6) (drill 0.3) (layers "F.Cu" "B.Cu") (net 6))
 (via (at 138.2 106.7) (size 0.6) (drill 0.3) (layers "F.Cu" "B.Cu") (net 6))
 (via (at 140.7 106.7) (size 0.6) (drill 0.3) (layers "F.Cu" "B.Cu") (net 6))
 (via (at 150 87.9) (size 0.6) (drill 0.3) (layers "F.Cu" "B.Cu") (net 6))
 (via (at 138.2 97.9) (size 0.6) (drill 0.3) (layers "F.Cu" "B.Cu") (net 6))
 (via (at 137.7 104.3) (size 0.6) (drill 0.3) (layers "F.Cu" "B.Cu") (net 6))
 (segment (start 140.1 96.8) (end 149 87.9) (width 0.2) (layer "B.Cu") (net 6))
 (segment (start 137.7 104.3) (end 137.7 98.4) (width 0.2) (layer "B.Cu") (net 6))
 (segment (start 140.7 106.7) (end 138.2 106.7) (width 0.2) (layer "B.Cu") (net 6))
 (segment (start 149 87.9) (end 150 87.9) (width 0.2) (layer "B.Cu") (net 6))
 (segment (start 137.7 98.4) (end 138.2 97.9) (width 0.2) (layer "B.Cu") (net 6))
 (segment (start 164.4125 113.5) (end 157.5625 106.65) (width 0.2) (layer "F.Cu") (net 4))
 (segment (start 158 103.8) (end 159.4375 102.3625) (width 0.2) (layer "F.Cu") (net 4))
 (segment (start 148.6625 96.6) (end 159.4375 96.6) (width 0.2) (layer "F.Cu") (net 4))
 (segment (start 147.5625 95.5) (end 148.6625 96.6) (width 0.2) (layer "F.Cu") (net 4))
 (segment (start 157.5625 105.5) (end 156.625 105.5) (width 0.2) (layer "F.Cu") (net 4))
 (segment (start 159.4375 102.3625) (end 159.4375 95.5) (width 0.2) (layer "F.Cu") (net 4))
 (segment (start 157.5625 106.65) (end 157.5625 105.5) (width 0.2) (layer "F.Cu") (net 4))
 (via (at 156.625 105.5) (size 0.6) (drill 0.3) (layers "F.Cu" "B.Cu") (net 4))
 (via (at 158 103.8) (size 0.6) (drill 0.3) (layers "F.Cu" "B.Cu") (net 4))
 (segment (start 156.625 105.5) (end 158 104.125) (width 0.2) (layer "B.Cu") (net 4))
 (segment (start 158 104.125) (end 158 103.8) (width 0.2) (layer "B.Cu") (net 4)))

